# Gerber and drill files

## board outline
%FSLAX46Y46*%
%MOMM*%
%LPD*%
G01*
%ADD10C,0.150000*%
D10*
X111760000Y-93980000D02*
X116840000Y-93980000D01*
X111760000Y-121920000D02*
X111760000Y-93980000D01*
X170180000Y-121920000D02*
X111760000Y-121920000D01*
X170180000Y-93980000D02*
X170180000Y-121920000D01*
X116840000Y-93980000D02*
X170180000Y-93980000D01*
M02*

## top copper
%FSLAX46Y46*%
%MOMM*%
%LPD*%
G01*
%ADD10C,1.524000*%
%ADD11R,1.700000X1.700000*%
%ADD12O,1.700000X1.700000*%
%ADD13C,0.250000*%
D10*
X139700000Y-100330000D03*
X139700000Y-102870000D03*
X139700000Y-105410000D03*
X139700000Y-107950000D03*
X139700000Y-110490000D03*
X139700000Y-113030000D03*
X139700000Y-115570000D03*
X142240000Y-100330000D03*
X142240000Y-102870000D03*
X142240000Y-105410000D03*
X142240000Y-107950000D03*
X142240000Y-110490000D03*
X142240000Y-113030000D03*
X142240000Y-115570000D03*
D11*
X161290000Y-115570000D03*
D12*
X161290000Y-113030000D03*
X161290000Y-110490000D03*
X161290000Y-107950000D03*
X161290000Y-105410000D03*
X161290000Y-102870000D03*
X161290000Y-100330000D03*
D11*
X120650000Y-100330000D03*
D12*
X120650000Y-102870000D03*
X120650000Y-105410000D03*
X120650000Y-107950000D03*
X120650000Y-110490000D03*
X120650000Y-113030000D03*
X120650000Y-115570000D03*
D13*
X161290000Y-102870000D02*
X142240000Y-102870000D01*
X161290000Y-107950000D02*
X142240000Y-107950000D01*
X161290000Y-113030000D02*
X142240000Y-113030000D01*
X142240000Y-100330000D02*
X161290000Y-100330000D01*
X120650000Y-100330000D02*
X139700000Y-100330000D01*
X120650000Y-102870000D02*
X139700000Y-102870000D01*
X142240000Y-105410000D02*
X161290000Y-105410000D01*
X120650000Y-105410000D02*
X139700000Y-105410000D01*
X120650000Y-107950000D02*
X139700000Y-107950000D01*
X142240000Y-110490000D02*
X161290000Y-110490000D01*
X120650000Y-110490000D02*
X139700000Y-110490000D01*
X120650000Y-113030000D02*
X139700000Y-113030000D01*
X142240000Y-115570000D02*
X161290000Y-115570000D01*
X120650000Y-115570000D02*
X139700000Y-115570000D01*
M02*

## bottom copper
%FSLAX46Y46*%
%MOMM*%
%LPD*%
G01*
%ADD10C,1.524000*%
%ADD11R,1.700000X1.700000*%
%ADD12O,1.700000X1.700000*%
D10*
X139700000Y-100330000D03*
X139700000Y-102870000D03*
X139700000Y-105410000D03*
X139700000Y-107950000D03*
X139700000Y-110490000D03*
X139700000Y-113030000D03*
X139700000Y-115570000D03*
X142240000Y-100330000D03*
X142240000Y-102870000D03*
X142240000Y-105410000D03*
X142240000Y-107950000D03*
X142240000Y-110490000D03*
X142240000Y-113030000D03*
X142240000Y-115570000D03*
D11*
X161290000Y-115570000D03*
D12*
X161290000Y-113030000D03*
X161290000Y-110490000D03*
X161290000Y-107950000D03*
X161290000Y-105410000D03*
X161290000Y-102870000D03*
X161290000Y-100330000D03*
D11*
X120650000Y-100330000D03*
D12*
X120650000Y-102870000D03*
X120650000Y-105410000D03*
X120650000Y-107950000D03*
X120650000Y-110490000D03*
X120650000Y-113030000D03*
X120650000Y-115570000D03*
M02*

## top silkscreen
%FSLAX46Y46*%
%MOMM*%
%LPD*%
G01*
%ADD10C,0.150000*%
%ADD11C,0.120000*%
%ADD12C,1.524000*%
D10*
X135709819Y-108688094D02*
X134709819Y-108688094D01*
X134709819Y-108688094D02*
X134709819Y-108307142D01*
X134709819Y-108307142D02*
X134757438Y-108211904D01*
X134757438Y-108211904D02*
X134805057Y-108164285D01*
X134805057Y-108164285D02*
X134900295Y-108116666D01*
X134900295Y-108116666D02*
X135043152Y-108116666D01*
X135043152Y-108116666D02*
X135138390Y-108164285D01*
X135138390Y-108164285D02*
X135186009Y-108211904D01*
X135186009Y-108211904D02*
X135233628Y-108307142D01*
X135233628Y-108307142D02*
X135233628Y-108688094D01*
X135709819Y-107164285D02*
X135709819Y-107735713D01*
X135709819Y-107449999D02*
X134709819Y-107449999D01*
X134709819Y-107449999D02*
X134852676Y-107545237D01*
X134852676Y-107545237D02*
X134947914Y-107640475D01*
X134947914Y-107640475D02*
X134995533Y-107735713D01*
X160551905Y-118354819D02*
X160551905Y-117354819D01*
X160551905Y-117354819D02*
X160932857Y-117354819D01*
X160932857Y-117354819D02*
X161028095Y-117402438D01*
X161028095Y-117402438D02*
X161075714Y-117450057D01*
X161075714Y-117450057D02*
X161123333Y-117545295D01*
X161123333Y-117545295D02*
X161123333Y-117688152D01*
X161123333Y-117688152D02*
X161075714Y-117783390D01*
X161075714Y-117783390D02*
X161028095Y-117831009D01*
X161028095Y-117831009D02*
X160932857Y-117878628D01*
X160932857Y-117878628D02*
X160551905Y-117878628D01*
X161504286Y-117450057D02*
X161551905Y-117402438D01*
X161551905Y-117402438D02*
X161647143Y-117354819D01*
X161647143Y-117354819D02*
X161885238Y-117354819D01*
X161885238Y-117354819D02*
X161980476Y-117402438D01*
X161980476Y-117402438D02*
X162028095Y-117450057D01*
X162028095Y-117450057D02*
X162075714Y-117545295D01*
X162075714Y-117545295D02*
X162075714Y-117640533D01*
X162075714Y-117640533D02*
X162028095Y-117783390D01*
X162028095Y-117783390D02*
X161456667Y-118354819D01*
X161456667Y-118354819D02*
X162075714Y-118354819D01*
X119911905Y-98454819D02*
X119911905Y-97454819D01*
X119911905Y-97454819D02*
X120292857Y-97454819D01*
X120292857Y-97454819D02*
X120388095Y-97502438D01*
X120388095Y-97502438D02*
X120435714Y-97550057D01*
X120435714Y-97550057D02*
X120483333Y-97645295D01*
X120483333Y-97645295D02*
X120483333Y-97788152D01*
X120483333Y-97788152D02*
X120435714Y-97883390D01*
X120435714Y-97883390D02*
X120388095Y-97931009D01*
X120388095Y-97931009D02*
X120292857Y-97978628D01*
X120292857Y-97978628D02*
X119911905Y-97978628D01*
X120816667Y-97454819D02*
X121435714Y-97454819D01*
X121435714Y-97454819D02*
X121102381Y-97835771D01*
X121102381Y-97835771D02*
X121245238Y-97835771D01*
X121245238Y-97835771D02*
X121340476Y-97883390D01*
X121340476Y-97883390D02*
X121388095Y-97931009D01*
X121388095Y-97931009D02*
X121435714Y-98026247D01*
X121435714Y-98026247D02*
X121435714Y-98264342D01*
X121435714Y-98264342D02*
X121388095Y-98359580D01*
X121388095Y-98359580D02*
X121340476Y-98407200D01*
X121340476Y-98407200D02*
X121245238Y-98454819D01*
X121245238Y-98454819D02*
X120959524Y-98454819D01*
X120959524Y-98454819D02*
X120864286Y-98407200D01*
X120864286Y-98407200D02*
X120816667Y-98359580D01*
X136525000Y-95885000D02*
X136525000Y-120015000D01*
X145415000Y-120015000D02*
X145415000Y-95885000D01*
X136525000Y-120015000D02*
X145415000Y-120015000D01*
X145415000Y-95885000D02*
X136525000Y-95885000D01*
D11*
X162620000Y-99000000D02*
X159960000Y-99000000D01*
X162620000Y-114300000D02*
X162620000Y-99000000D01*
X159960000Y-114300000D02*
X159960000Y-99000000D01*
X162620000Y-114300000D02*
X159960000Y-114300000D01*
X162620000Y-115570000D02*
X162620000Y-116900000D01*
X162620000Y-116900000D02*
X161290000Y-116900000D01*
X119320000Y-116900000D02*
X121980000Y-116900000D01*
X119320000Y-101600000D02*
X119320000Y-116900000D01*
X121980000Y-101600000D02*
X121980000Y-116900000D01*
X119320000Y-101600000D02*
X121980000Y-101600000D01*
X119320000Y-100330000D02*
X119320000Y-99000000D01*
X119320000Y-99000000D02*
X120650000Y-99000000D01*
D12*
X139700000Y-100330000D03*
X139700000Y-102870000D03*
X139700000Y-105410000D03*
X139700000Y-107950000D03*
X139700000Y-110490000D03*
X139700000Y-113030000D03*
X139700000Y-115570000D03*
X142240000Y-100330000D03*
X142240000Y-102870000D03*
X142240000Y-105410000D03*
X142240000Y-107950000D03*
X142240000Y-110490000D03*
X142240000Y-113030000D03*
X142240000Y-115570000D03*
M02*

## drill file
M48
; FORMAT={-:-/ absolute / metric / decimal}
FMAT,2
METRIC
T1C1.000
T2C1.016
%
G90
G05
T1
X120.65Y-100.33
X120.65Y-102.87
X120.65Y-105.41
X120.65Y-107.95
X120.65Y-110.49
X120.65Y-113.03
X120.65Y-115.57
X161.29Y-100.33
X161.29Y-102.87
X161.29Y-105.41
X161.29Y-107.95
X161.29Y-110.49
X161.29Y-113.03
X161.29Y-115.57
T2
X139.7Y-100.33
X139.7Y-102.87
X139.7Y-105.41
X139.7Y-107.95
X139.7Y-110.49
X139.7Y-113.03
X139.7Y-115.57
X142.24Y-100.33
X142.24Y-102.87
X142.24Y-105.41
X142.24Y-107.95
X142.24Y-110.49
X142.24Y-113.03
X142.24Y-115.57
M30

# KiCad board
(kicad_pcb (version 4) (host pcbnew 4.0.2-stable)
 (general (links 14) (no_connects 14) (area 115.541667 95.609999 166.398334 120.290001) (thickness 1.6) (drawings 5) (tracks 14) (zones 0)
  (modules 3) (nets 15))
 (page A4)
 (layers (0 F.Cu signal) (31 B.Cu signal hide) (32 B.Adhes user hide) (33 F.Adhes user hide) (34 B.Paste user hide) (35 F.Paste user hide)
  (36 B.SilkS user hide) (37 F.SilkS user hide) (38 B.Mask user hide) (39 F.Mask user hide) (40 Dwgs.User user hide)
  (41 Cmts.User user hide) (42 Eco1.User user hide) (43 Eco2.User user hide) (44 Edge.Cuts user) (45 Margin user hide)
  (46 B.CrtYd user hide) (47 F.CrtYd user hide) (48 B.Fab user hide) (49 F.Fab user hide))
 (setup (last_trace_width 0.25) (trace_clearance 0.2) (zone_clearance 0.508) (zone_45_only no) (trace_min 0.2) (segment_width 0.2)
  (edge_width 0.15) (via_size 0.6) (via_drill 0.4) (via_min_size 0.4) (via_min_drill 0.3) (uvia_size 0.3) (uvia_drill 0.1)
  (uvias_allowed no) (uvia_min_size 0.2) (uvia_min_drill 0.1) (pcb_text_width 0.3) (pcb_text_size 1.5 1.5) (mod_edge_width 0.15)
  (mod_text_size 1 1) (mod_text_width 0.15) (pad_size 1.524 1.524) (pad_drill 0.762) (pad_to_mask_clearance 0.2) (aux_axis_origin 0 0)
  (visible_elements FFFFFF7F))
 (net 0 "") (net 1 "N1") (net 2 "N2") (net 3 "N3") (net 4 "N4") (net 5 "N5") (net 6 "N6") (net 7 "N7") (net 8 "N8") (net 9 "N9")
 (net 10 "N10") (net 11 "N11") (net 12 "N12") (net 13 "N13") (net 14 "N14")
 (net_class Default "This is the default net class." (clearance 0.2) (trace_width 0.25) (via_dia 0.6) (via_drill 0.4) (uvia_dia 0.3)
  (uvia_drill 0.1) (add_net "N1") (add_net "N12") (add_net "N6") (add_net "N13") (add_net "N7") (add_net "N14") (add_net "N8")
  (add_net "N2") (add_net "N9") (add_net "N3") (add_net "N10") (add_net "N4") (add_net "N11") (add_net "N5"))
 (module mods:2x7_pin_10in (layer F.Cu) (at 140.97 107.95 270)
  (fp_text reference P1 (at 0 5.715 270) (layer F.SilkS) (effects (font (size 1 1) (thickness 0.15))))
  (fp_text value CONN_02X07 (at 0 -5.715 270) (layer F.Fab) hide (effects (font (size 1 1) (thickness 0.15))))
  (fp_line (start -12.065 4.445) (end 12.065 4.445) (layer F.SilkS) (width 0.15))
  (fp_line (start 12.065 -4.445) (end -12.065 -4.445) (layer F.SilkS) (width 0.15))
  (fp_line (start 12.065 4.445) (end 12.065 -4.445) (layer F.SilkS) (width 0.15))
  (fp_line (start -12.065 -4.445) (end -12.065 4.445) (layer F.SilkS) (width 0.15))
  (pad 1 thru_hole circle (at -7.62 1.27 270) (size 1.524 1.524) (drill 1.016) (layers *.Cu *.Mask F.SilkS) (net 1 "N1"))
  (pad 3 thru_hole circle (at -5.08 1.27 270) (size 1.524 1.524) (drill 1.016) (layers *.Cu *.Mask F.SilkS) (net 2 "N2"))
  (pad 5 thru_hole circle (at -2.54 1.27 270) (size 1.524 1.524) (drill 1.016) (layers *.Cu *.Mask F.SilkS) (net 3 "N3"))
  (pad 7 thru_hole circle (at 0 1.27 270) (size 1.524 1.524) (drill 1.016) (layers *.Cu *.Mask F.SilkS) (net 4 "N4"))
  (pad 9 thru_hole circle (at 2.54 1.27 270) (size 1.524 1.524) (drill 1.016) (layers *.Cu *.Mask F.SilkS) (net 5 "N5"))
  (pad 11 thru_hole circle (at 5.08 1.27 270) (size 1.524 1.524) (drill 1.016) (layers *.Cu *.Mask F.SilkS) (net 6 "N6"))
  (pad 13 thru_hole circle (at 7.62 1.27 270) (size 1.524 1.524) (drill 1.016) (layers *.Cu *.Mask F.SilkS) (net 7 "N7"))
  (pad 2 thru_hole circle (at -7.62 -1.27 270) (size 1.524 1.524) (drill 1.016) (layers *.Cu *.Mask F.SilkS) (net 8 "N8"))
  (pad 4 thru_hole circle (at -5.08 -1.27 270) (size 1.524 1.524) (drill 1.016) (layers *.Cu *.Mask F.SilkS) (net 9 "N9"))
  (pad 6 thru_hole circle (at -2.54 -1.27 270) (size 1.524 1.524) (drill 1.016) (layers *.Cu *.Mask F.SilkS) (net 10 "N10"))
  (pad 8 thru_hole circle (at 0 -1.27 270) (size 1.524 1.524) (drill 1.016) (layers *.Cu *.Mask F.SilkS) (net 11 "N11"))
  (pad 10 thru_hole circle (at 2.54 -1.27 270) (size 1.524 1.524) (drill 1.016) (layers *.Cu *.Mask F.SilkS) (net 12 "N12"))
  (pad 12 thru_hole circle (at 5.08 -1.27 270) (size 1.524 1.524) (drill 1.016) (layers *.Cu *.Mask F.SilkS) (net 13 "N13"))
  (pad 14 thru_hole circle (at 7.62 -1.27 270) (size 1.524 1.524) (drill 1.016) (layers *.Cu *.Mask F.SilkS) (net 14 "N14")))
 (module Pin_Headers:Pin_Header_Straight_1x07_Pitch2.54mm (layer F.Cu) (at 161.29 115.57 180)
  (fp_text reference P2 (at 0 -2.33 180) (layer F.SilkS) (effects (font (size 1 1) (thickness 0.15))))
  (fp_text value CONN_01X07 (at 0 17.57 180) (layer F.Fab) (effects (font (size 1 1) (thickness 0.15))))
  (fp_line (start -1.33 16.57) (end 1.33 16.57) (layer F.SilkS) (width 0.12))
  (fp_line (start -1.33 1.27) (end -1.33 16.57) (layer F.SilkS) (width 0.12))
  (fp_line (start 1.33 1.27) (end 1.33 16.57) (layer F.SilkS) (width 0.12))
  (fp_line (start -1.33 1.27) (end 1.33 1.27) (layer F.SilkS) (width 0.12))
  (fp_line (start -1.33 0) (end -1.33 -1.33) (layer F.SilkS) (width 0.12))
  (fp_line (start -1.33 -1.33) (end 0 -1.33) (layer F.SilkS) (width 0.12))
  (pad 1 thru_hole rect (at 0 0 180) (size 1.7 1.7) (drill 1) (layers *.Cu *.Mask) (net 7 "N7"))
  (pad 2 thru_hole oval (at 0 2.54 180) (size 1.7 1.7) (drill 1) (layers *.Cu *.Mask) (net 6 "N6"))
  (pad 3 thru_hole oval (at 0 5.08 180) (size 1.7 1.7) (drill 1) (layers *.Cu *.Mask) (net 5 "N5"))
  (pad 4 thru_hole oval (at 0 7.62 180) (size 1.7 1.7) (drill 1) (layers *.Cu *.Mask) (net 4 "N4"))
  (pad 5 thru_hole oval (at 0 10.16 180) (size 1.7 1.7) (drill 1) (layers *.Cu *.Mask) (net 3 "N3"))
  (pad 6 thru_hole oval (at 0 12.7 180) (size 1.7 1.7) (drill 1) (layers *.Cu *.Mask) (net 2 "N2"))
  (pad 7 thru_hole oval (at 0 15.24 180) (size 1.7 1.7) (drill 1) (layers *.Cu *.Mask) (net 1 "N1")))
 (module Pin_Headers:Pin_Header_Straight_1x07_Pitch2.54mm (layer F.Cu) (at 120.65 100.33)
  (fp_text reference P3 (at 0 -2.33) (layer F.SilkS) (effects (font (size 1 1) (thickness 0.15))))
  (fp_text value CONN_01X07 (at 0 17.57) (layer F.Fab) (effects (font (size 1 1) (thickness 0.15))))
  (fp_line (start -1.33 16.57) (end 1.33 16.57) (layer F.SilkS) (width 0.12))
  (fp_line (start -1.33 1.27) (end -1.33 16.57) (layer F.SilkS) (width 0.12))
  (fp_line (start 1.33 1.27) (end 1.33 16.57) (layer F.SilkS) (width 0.12))
  (fp_line (start -1.33 1.27) (end 1.33 1.27) (layer F.SilkS) (width 0.12))
  (fp_line (start -1.33 0) (end -1.33 -1.33) (layer F.SilkS) (width 0.12))
  (fp_line (start -1.33 -1.33) (end 0 -1.33) (layer F.SilkS) (width 0.12))
  (pad 1 thru_hole rect (at 0 0) (size 1.7 1.7) (drill 1) (layers *.Cu *.Mask) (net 8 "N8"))
  (pad 2 thru_hole oval (at 0 2.54) (size 1.7 1.7) (drill 1) (layers *.Cu *.Mask) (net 9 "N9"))
  (pad 3 thru_hole oval (at 0 5.08) (size 1.7 1.7) (drill 1) (layers *.Cu *.Mask) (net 10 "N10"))
  (pad 4 thru_hole oval (at 0 7.62) (size 1.7 1.7) (drill 1) (layers *.Cu *.Mask) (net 11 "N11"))
  (pad 5 thru_hole oval (at 0 10.16) (size 1.7 1.7) (drill 1) (layers *.Cu *.Mask) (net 12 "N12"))
  (pad 6 thru_hole oval (at 0 12.7) (size 1.7 1.7) (drill 1) (layers *.Cu *.Mask) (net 13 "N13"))
  (pad 7 thru_hole oval (at 0 15.24) (size 1.7 1.7) (drill 1) (layers *.Cu *.Mask) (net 14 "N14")))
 (gr_line (start 111.76 93.98) (end 116.84 93.98) (angle 90) (layer Edge.Cuts) (width 0.15))
 (gr_line (start 111.76 121.92) (end 111.76 93.98) (angle 90) (layer Edge.Cuts) (width 0.15))
 (gr_line (start 170.18 121.92) (end 111.76 121.92) (angle 90) (layer Edge.Cuts) (width 0.15))
 (gr_line (start 170.18 93.98) (end 170.18 121.92) (angle 90) (layer Edge.Cuts) (width 0.15))
 (gr_line (start 116.84 93.98) (end 170.18 93.98) (angle 90) (layer Edge.Cuts) (width 0.15))
 (segment (start 161.29 102.87) (end 142.24 102.87) (width 0.25) (layer F.Cu) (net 2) (status C00000))
 (segment (start 161.29 107.95) (end 142.24 107.95) (width 0.25) (layer F.Cu) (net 4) (status C00000))
 (segment (start 161.29 113.03) (end 142.24 113.03) (width 0.25) (layer F.Cu) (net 6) (status C00000))
 (segment (start 142.24 100.33) (end 161.29 100.33) (width 0.25) (layer F.Cu) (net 8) (status C00000))
 (segment (start 120.65 100.33) (end 139.7 100.33) (width 0.25) (layer F.Cu) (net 8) (status C00000))
 (segment (start 120.65 102.87) (end 139.7 102.87) (width 0.25) (layer F.Cu) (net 9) (status C00000))
 (segment (start 142.24 105.41) (end 161.29 105.41) (width 0.25) (layer F.Cu) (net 10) (status C00000))
 (segment (start 120.65 105.41) (end 139.7 105.41) (width 0.25) (layer F.Cu) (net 10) (status C00000))
 (segment (start 120.65 107.95) (end 139.7 107.95) (width 0.25) (layer F.Cu) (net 11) (status C00000))
 (segment (start 142.24 110.49) (end 161.29 110.49) (width 0.25) (layer F.Cu) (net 12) (status C00000))
 (segment (start 120.65 110.49) (end 139.7 110.49) (width 0.25) (layer F.Cu) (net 12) (status C00000))
 (segment (start 120.65 113.03) (end 139.7 113.03) (width 0.25) (layer F.Cu) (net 13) (status C00000))
 (segment (start 142.24 115.57) (end 161.29 115.57) (width 0.25) (layer F.Cu) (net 14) (status C00000))
 (segment (start 120.65 115.57) (end 139.7 115.57) (width 0.25) (layer F.Cu) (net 14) (status C00000)))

